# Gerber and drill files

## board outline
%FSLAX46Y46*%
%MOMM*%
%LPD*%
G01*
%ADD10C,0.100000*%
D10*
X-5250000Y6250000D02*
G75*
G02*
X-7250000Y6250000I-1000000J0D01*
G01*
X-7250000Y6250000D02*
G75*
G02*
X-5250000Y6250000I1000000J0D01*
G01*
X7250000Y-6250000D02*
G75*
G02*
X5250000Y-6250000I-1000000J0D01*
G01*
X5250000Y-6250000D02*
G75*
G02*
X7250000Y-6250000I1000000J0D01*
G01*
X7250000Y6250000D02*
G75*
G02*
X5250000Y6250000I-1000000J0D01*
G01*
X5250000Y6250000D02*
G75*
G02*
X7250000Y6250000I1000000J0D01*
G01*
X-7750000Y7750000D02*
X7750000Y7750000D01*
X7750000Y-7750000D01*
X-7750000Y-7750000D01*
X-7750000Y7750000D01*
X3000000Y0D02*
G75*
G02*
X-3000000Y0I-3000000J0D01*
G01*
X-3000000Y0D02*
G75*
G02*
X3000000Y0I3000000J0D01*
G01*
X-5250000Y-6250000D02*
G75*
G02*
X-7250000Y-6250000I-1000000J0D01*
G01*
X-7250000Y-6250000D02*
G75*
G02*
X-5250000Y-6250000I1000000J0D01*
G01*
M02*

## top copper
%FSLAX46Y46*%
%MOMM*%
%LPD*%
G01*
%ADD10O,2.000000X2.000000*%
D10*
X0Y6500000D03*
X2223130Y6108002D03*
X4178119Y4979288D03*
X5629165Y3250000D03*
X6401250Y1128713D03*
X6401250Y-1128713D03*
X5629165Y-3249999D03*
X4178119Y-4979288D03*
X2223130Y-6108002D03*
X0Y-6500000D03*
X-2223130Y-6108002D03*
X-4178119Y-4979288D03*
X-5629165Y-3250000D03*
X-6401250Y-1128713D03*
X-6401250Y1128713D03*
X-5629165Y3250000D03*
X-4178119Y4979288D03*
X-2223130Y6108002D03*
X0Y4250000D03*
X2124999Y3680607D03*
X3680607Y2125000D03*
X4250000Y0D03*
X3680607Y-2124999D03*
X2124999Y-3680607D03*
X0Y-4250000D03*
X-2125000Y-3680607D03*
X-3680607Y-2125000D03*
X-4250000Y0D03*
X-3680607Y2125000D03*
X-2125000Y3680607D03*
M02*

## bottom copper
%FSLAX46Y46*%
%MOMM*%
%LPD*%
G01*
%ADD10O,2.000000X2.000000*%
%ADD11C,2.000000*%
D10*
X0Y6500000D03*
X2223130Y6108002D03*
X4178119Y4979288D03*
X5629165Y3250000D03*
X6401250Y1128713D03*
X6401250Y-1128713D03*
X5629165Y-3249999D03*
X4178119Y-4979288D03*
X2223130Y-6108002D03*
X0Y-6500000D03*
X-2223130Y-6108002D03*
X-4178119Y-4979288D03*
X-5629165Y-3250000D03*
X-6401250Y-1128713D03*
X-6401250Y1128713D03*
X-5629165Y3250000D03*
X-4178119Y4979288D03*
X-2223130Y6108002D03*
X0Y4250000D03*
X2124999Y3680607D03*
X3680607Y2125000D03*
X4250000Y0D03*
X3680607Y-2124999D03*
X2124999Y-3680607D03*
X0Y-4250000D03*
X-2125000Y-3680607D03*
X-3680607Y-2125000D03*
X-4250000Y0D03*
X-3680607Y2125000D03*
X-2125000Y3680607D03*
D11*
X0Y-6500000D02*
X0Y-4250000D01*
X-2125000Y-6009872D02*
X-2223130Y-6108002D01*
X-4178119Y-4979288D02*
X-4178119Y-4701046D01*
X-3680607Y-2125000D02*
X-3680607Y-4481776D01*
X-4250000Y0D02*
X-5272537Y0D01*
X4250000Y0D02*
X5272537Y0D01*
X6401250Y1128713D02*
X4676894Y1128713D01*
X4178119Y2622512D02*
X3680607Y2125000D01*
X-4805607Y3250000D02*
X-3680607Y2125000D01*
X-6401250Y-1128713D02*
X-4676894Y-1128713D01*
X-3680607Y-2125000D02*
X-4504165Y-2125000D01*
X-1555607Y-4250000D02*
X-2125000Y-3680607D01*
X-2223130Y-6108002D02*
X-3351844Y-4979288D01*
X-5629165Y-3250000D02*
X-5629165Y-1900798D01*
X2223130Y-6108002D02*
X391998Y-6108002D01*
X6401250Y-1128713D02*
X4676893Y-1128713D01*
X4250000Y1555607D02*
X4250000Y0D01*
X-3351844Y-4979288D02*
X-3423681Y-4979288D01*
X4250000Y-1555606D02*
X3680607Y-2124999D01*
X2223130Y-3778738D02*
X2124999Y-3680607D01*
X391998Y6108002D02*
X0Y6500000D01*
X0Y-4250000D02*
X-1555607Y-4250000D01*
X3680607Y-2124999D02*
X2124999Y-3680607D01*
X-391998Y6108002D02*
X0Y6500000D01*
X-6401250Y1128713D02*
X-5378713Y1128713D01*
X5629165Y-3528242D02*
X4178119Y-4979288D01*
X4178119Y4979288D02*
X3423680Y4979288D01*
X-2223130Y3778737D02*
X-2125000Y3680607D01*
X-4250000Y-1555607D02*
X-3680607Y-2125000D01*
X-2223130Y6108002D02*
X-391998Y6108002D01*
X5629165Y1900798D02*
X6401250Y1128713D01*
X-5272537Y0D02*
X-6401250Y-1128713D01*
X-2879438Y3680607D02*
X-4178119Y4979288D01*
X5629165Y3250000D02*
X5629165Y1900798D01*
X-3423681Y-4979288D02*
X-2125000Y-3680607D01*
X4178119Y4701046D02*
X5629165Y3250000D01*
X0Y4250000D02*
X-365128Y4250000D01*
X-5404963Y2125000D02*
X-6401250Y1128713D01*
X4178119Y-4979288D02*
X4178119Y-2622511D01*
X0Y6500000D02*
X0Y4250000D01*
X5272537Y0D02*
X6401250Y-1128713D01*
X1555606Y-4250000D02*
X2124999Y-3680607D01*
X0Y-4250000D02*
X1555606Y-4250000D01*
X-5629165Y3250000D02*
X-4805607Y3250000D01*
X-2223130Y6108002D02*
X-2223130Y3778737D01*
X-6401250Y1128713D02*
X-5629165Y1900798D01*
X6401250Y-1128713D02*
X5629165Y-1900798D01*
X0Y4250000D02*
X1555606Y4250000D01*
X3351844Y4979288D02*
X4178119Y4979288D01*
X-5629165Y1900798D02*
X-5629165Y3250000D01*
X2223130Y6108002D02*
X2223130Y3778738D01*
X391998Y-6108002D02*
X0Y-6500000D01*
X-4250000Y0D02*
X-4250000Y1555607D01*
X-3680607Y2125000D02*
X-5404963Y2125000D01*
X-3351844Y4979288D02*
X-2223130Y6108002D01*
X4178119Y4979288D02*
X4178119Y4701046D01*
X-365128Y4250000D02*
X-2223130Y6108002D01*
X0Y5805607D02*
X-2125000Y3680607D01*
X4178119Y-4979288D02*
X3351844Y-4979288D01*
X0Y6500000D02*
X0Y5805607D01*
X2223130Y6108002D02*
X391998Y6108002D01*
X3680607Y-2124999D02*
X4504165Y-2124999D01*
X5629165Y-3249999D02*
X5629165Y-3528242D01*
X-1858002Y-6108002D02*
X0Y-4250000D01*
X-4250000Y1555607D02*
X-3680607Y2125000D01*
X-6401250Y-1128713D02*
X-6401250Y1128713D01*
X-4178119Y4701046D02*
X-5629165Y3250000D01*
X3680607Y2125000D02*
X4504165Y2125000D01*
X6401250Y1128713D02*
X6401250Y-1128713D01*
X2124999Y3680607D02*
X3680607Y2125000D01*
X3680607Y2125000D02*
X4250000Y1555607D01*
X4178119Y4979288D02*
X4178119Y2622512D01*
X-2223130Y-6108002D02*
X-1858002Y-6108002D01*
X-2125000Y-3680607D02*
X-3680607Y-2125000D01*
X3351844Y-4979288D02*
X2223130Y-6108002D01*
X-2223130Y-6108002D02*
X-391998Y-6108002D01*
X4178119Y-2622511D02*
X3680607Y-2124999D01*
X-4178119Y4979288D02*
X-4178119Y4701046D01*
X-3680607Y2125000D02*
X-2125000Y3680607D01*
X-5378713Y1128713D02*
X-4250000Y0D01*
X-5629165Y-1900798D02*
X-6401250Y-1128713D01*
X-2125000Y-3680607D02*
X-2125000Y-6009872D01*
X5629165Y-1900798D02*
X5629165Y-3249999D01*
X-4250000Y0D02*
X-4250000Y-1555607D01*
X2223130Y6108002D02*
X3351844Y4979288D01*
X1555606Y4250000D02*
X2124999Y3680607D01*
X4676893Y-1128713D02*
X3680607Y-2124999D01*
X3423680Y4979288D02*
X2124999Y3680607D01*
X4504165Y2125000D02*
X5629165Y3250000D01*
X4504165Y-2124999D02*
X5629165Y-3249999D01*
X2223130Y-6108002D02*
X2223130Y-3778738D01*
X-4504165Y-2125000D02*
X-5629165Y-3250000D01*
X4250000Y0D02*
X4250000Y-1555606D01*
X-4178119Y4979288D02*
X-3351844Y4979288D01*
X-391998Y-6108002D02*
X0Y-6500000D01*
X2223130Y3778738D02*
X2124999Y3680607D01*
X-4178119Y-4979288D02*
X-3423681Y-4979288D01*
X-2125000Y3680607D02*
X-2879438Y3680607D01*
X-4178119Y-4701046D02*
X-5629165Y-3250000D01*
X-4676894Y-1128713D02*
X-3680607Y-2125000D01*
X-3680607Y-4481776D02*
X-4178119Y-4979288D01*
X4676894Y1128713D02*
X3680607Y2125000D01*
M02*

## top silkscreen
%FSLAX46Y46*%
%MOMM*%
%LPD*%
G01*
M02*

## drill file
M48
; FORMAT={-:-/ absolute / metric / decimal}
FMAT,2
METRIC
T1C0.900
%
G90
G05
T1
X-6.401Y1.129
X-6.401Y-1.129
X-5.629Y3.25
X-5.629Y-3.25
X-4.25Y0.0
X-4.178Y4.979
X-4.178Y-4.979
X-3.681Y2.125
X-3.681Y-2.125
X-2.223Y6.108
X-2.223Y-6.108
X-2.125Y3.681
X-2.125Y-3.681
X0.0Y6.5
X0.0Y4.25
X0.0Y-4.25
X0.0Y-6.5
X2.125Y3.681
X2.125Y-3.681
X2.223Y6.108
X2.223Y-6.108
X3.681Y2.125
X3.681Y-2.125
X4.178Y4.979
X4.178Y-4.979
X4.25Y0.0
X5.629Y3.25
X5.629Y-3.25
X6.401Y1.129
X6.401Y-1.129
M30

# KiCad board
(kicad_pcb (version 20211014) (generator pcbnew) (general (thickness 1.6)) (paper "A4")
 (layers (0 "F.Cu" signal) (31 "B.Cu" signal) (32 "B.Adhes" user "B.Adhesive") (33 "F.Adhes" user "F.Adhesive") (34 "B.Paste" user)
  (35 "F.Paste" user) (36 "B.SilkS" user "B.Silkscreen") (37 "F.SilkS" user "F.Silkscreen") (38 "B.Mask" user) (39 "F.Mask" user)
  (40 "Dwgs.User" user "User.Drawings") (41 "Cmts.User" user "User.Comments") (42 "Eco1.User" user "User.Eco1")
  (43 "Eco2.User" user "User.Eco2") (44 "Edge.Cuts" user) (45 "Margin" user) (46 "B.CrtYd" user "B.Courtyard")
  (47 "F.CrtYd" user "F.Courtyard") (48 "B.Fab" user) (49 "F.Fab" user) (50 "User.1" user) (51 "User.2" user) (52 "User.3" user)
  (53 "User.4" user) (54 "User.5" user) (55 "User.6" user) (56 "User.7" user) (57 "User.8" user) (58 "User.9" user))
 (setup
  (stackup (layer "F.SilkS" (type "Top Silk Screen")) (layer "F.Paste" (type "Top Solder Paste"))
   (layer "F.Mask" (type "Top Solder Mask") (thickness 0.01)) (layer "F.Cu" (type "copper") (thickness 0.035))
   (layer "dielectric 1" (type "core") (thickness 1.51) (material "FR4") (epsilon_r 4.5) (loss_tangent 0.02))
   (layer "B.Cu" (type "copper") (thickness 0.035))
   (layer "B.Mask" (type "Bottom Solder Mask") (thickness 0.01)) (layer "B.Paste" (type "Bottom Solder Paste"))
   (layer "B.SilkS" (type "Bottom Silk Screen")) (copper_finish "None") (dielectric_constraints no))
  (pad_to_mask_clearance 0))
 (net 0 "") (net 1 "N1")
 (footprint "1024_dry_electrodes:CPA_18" (layer "F.Cu") (at 0 0)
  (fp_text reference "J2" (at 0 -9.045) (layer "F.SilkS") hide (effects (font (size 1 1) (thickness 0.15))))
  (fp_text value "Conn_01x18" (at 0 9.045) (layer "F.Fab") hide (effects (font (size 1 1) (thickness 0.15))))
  (pad "1" thru_hole oval (at 0 -6.5) (size 2 2) (drill 0.9) (layers *.Cu *.Mask) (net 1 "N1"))
  (pad "2" thru_hole oval (at 2.22313 -6.108002) (size 2 2) (drill 0.9) (layers *.Cu *.Mask) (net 1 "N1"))
  (pad "3" thru_hole oval (at 4.178119 -4.979288) (size 2 2) (drill 0.9) (layers *.Cu *.Mask) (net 1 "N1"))
  (pad "4" thru_hole oval (at 5.629165 -3.25) (size 2 2) (drill 0.9) (layers *.Cu *.Mask) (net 1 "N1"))
  (pad "5" thru_hole oval (at 6.40125 -1.128713) (size 2 2) (drill 0.9) (layers *.Cu *.Mask) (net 1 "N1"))
  (pad "6" thru_hole oval (at 6.40125 1.128713) (size 2 2) (drill 0.9) (layers *.Cu *.Mask) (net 1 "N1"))
  (pad "7" thru_hole oval (at 5.629165 3.249999) (size 2 2) (drill 0.9) (layers *.Cu *.Mask) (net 1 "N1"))
  (pad "8" thru_hole oval (at 4.178119 4.979288) (size 2 2) (drill 0.9) (layers *.Cu *.Mask) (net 1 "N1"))
  (pad "9" thru_hole oval (at 2.22313 6.108002) (size 2 2) (drill 0.9) (layers *.Cu *.Mask) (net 1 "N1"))
  (pad "10" thru_hole oval (at 0 6.5) (size 2 2) (drill 0.9) (layers *.Cu *.Mask) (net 1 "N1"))
  (pad "11" thru_hole oval (at -2.22313 6.108002) (size 2 2) (drill 0.9) (layers *.Cu *.Mask) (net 1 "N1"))
  (pad "12" thru_hole oval (at -4.178119 4.979288) (size 2 2) (drill 0.9) (layers *.Cu *.Mask) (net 1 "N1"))
  (pad "13" thru_hole oval (at -5.629165 3.25) (size 2 2) (drill 0.9) (layers *.Cu *.Mask) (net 1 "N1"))
  (pad "14" thru_hole oval (at -6.40125 1.128713) (size 2 2) (drill 0.9) (layers *.Cu *.Mask) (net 1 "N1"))
  (pad "15" thru_hole oval (at -6.40125 -1.128713) (size 2 2) (drill 0.9) (layers *.Cu *.Mask) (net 1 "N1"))
  (pad "16" thru_hole oval (at -5.629165 -3.25) (size 2 2) (drill 0.9) (layers *.Cu *.Mask) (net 1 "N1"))
  (pad "17" thru_hole oval (at -4.178119 -4.979288) (size 2 2) (drill 0.9) (layers *.Cu *.Mask) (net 1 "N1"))
  (pad "18" thru_hole oval (at -2.22313 -6.108002) (size 2 2) (drill 0.9) (layers *.Cu *.Mask) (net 1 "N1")))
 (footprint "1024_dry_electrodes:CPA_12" (layer "F.Cu") (at 0 0)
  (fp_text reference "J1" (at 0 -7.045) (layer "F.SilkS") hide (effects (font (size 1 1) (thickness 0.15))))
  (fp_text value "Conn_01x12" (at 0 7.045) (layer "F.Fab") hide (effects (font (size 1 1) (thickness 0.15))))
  (pad "1" thru_hole oval (at 0 -4.25) (size 2 2) (drill 0.9) (layers *.Cu *.Mask) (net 1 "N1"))
  (pad "2" thru_hole oval (at 2.124999 -3.680607) (size 2 2) (drill 0.9) (layers *.Cu *.Mask) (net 1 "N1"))
  (pad "3" thru_hole oval (at 3.680607 -2.125) (size 2 2) (drill 0.9) (layers *.Cu *.Mask) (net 1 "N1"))
  (pad "4" thru_hole oval (at 4.25 0) (size 2 2) (drill 0.9) (layers *.Cu *.Mask) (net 1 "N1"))
  (pad "5" thru_hole oval (at 3.680607 2.124999) (size 2 2) (drill 0.9) (layers *.Cu *.Mask) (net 1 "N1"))
  (pad "6" thru_hole oval (at 2.124999 3.680607) (size 2 2) (drill 0.9) (layers *.Cu *.Mask) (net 1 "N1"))
  (pad "7" thru_hole oval (at 0 4.25) (size 2 2) (drill 0.9) (layers *.Cu *.Mask) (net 1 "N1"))
  (pad "8" thru_hole oval (at -2.125 3.680607) (size 2 2) (drill 0.9) (layers *.Cu *.Mask) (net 1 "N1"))
  (pad "9" thru_hole oval (at -3.680607 2.125) (size 2 2) (drill 0.9) (layers *.Cu *.Mask) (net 1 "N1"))
  (pad "10" thru_hole oval (at -4.25 0) (size 2 2) (drill 0.9) (layers *.Cu *.Mask) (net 1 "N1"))
  (pad "11" thru_hole oval (at -3.680607 -2.125) (size 2 2) (drill 0.9) (layers *.Cu *.Mask) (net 1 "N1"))
  (pad "12" thru_hole oval (at -2.125 -3.680607) (size 2 2) (drill 0.9) (layers *.Cu *.Mask) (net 1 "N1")))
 (gr_circle (center -6.25 -6.25) (end -5.25 -6.25) (layer "Edge.Cuts") (width 0.1) (fill none))
 (gr_circle (center 6.25 6.25) (end 7.25 6.25) (layer "Edge.Cuts") (width 0.1) (fill none))
 (gr_circle (center 6.25 -6.25) (end 7.25 -6.25) (layer "Edge.Cuts") (width 0.1) (fill none))
 (gr_rect (start 7.75 7.75) (end -7.75 -7.75) (layer "Edge.Cuts") (width 0.1) (fill none))
 (gr_circle (center 0 0) (end 3 0) (layer "Edge.Cuts") (width 0.1) (fill none))
 (gr_circle (center -6.25 6.25) (end -5.25 6.25) (layer "Edge.Cuts") (width 0.1) (fill none))
 (segment (start 0 6.5) (end 0 4.25) (width 2) (layer "B.Cu") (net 1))
 (segment (start -2.125 6.009872) (end -2.22313 6.108002) (width 2) (layer "B.Cu") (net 1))
 (segment (start -4.178119 4.979288) (end -4.178119 4.701046) (width 2) (layer "B.Cu") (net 1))
 (segment (start -3.680607 2.125) (end -3.680607 4.481776) (width 2) (layer "B.Cu") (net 1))
 (segment (start -4.25 0) (end -5.272537 0) (width 2) (layer "B.Cu") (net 1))
 (segment (start 4.25 0) (end 5.272537 0) (width 2) (layer "B.Cu") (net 1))
 (segment (start 6.40125 -1.128713) (end 4.676894 -1.128713) (width 2) (layer "B.Cu") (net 1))
 (segment (start 4.178119 -2.622512) (end 3.680607 -2.125) (width 2) (layer "B.Cu") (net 1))
 (segment (start -4.805607 -3.25) (end -3.680607 -2.125) (width 2) (layer "B.Cu") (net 1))
 (segment (start -6.40125 1.128713) (end -4.676894 1.128713) (width 2) (layer "B.Cu") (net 1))
 (segment (start -3.680607 2.125) (end -4.504165 2.125) (width 2) (layer "B.Cu") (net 1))
 (segment (start -1.555607 4.25) (end -2.125 3.680607) (width 2) (layer "B.Cu") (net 1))
 (segment (start -2.22313 6.108002) (end -3.351844 4.979288) (width 2) (layer "B.Cu") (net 1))
 (segment (start -5.629165 3.25) (end -5.629165 1.900798) (width 2) (layer "B.Cu") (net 1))
 (segment (start 2.22313 6.108002) (end 0.391998 6.108002) (width 2) (layer "B.Cu") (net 1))
 (segment (start 6.40125 1.128713) (end 4.676893 1.128713) (width 2) (layer "B.Cu") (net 1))
 (segment (start 4.25 -1.555607) (end 4.25 0) (width 2) (layer "B.Cu") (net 1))
 (segment (start -3.351844 4.979288) (end -3.423681 4.979288) (width 2) (layer "B.Cu") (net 1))
 (segment (start 4.25 1.555606) (end 3.680607 2.124999) (width 2) (layer "B.Cu") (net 1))
 (segment (start 2.22313 3.778738) (end 2.124999 3.680607) (width 2) (layer "B.Cu") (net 1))
 (segment (start 0.391998 -6.108002) (end 0 -6.5) (width 2) (layer "B.Cu") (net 1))
 (segment (start 0 4.25) (end -1.555607 4.25) (width 2) (layer "B.Cu") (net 1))
 (segment (start 3.680607 2.124999) (end 2.124999 3.680607) (width 2) (layer "B.Cu") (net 1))
 (segment (start -0.391998 -6.108002) (end 0 -6.5) (width 2) (layer "B.Cu") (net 1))
 (segment (start -6.40125 -1.128713) (end -5.378713 -1.128713) (width 2) (layer "B.Cu") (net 1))
 (segment (start 5.629165 3.528242) (end 4.178119 4.979288) (width 2) (layer "B.Cu") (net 1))
 (segment (start 4.178119 -4.979288) (end 3.42368 -4.979288) (width 2) (layer "B.Cu") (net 1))
 (segment (start -2.22313 -3.778737) (end -2.125 -3.680607) (width 2) (layer "B.Cu") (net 1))
 (segment (start -4.25 1.555607) (end -3.680607 2.125) (width 2) (layer "B.Cu") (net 1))
 (segment (start -2.22313 -6.108002) (end -0.391998 -6.108002) (width 2) (layer "B.Cu") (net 1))
 (segment (start 5.629165 -1.900798) (end 6.40125 -1.128713) (width 2) (layer "B.Cu") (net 1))
 (segment (start -5.272537 0) (end -6.40125 1.128713) (width 2) (layer "B.Cu") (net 1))
 (segment (start -2.879438 -3.680607) (end -4.178119 -4.979288) (width 2) (layer "B.Cu") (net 1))
 (segment (start 5.629165 -3.25) (end 5.629165 -1.900798) (width 2) (layer "B.Cu") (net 1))
 (segment (start -3.423681 4.979288) (end -2.125 3.680607) (width 2) (layer "B.Cu") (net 1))
 (segment (start 4.178119 -4.701046) (end 5.629165 -3.25) (width 2) (layer "B.Cu") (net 1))
 (segment (start 0 -4.25) (end -0.365128 -4.25) (width 2) (layer "B.Cu") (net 1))
 (segment (start -5.404963 -2.125) (end -6.40125 -1.128713) (width 2) (layer "B.Cu") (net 1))
 (segment (start 4.178119 4.979288) (end 4.178119 2.622511) (width 2) (layer "B.Cu") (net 1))
 (segment (start 0 -6.5) (end 0 -4.25) (width 2) (layer "B.Cu") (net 1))
 (segment (start 5.272537 0) (end 6.40125 1.128713) (width 2) (layer "B.Cu") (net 1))
 (segment (start 1.555606 4.25) (end 2.124999 3.680607) (width 2) (layer "B.Cu") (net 1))
 (segment (start 0 4.25) (end 1.555606 4.25) (width 2) (layer "B.Cu") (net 1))
 (segment (start -5.629165 -3.25) (end -4.805607 -3.25) (width 2) (layer "B.Cu") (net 1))
 (segment (start -2.22313 -6.108002) (end -2.22313 -3.778737) (width 2) (layer "B.Cu") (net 1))
 (segment (start -6.40125 -1.128713) (end -5.629165 -1.900798) (width 2) (layer "B.Cu") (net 1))
 (segment (start 6.40125 1.128713) (end 5.629165 1.900798) (width 2) (layer "B.Cu") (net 1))
 (segment (start 0 -4.25) (end 1.555606 -4.25) (width 2) (layer "B.Cu") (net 1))
 (segment (start 3.351844 -4.979288) (end 4.178119 -4.979288) (width 2) (layer "B.Cu") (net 1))
 (segment (start -5.629165 -1.900798) (end -5.629165 -3.25) (width 2) (layer "B.Cu") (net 1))
 (segment (start 2.22313 -6.108002) (end 2.22313 -3.778738) (width 2) (layer "B.Cu") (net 1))
 (segment (start 0.391998 6.108002) (end 0 6.5) (width 2) (layer "B.Cu") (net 1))
 (segment (start -4.25 0) (end -4.25 -1.555607) (width 2) (layer "B.Cu") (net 1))
 (segment (start -3.680607 -2.125) (end -5.404963 -2.125) (width 2) (layer "B.Cu") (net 1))
 (segment (start -3.351844 -4.979288) (end -2.22313 -6.108002) (width 2) (layer "B.Cu") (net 1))
 (segment (start 4.178119 -4.979288) (end 4.178119 -4.701046) (width 2) (layer "B.Cu") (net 1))
 (segment (start -0.365128 -4.25) (end -2.22313 -6.108002) (width 2) (layer "B.Cu") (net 1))
 (segment (start 0 -5.805607) (end -2.125 -3.680607) (width 2) (layer "B.Cu") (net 1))
 (segment (start 4.178119 4.979288) (end 3.351844 4.979288) (width 2) (layer "B.Cu") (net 1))
 (segment (start 0 -6.5) (end 0 -5.805607) (width 2) (layer "B.Cu") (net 1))
 (segment (start 2.22313 -6.108002) (end 0.391998 -6.108002) (width 2) (layer "B.Cu") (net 1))
 (segment (start 3.680607 2.124999) (end 4.504165 2.124999) (width 2) (layer "B.Cu") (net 1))
 (segment (start 5.629165 3.249999) (end 5.629165 3.528242) (width 2) (layer "B.Cu") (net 1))
 (segment (start -1.858002 6.108002) (end 0 4.25) (width 2) (layer "B.Cu") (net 1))
 (segment (start -4.25 -1.555607) (end -3.680607 -2.125) (width 2) (layer "B.Cu") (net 1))
 (segment (start -6.40125 1.128713) (end -6.40125 -1.128713) (width 2) (layer "B.Cu") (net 1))
 (segment (start -4.178119 -4.701046) (end -5.629165 -3.25) (width 2) (layer "B.Cu") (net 1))
 (segment (start 3.680607 -2.125) (end 4.504165 -2.125) (width 2) (layer "B.Cu") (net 1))
 (segment (start 6.40125 -1.128713) (end 6.40125 1.128713) (width 2) (layer "B.Cu") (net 1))
 (segment (start 2.124999 -3.680607) (end 3.680607 -2.125) (width 2) (layer "B.Cu") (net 1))
 (segment (start 3.680607 -2.125) (end 4.25 -1.555607) (width 2) (layer "B.Cu") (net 1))
 (segment (start 4.178119 -4.979288) (end 4.178119 -2.622512) (width 2) (layer "B.Cu") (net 1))
 (segment (start -2.22313 6.108002) (end -1.858002 6.108002) (width 2) (layer "B.Cu") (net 1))
 (segment (start -2.125 3.680607) (end -3.680607 2.125) (width 2) (layer "B.Cu") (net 1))
 (segment (start 3.351844 4.979288) (end 2.22313 6.108002) (width 2) (layer "B.Cu") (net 1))
 (segment (start -2.22313 6.108002) (end -0.391998 6.108002) (width 2) (layer "B.Cu") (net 1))
 (segment (start 4.178119 2.622511) (end 3.680607 2.124999) (width 2) (layer "B.Cu") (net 1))
 (segment (start -4.178119 -4.979288) (end -4.178119 -4.701046) (width 2) (layer "B.Cu") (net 1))
 (segment (start -3.680607 -2.125) (end -2.125 -3.680607) (width 2) (layer "B.Cu") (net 1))
 (segment (start -5.378713 -1.128713) (end -4.25 0) (width 2) (layer "B.Cu") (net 1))
 (segment (start -5.629165 1.900798) (end -6.40125 1.128713) (width 2) (layer "B.Cu") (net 1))
 (segment (start -2.125 3.680607) (end -2.125 6.009872) (width 2) (layer "B.Cu") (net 1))
 (segment (start 5.629165 1.900798) (end 5.629165 3.249999) (width 2) (layer "B.Cu") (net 1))
 (segment (start -4.25 0) (end -4.25 1.555607) (width 2) (layer "B.Cu") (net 1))
 (segment (start 2.22313 -6.108002) (end 3.351844 -4.979288) (width 2) (layer "B.Cu") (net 1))
 (segment (start 1.555606 -4.25) (end 2.124999 -3.680607) (width 2) (layer "B.Cu") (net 1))
 (segment (start 4.676893 1.128713) (end 3.680607 2.124999) (width 2) (layer "B.Cu") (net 1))
 (segment (start 3.42368 -4.979288) (end 2.124999 -3.680607) (width 2) (layer "B.Cu") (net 1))
 (segment (start 4.504165 -2.125) (end 5.629165 -3.25) (width 2) (layer "B.Cu") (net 1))
 (segment (start 4.504165 2.124999) (end 5.629165 3.249999) (width 2) (layer "B.Cu") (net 1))
 (segment (start 2.22313 6.108002) (end 2.22313 3.778738) (width 2) (layer "B.Cu") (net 1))
 (segment (start -4.504165 2.125) (end -5.629165 3.25) (width 2) (layer "B.Cu") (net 1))
 (segment (start 4.25 0) (end 4.25 1.555606) (width 2) (layer "B.Cu") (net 1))
 (segment (start -4.178119 -4.979288) (end -3.351844 -4.979288) (width 2) (layer "B.Cu") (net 1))
 (segment (start -0.391998 6.108002) (end 0 6.5) (width 2) (layer "B.Cu") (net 1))
 (segment (start 2.22313 -3.778738) (end 2.124999 -3.680607) (width 2) (layer "B.Cu") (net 1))
 (segment (start -4.178119 4.979288) (end -3.423681 4.979288) (width 2) (layer "B.Cu") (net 1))
 (segment (start -2.125 -3.680607) (end -2.879438 -3.680607) (width 2) (layer "B.Cu") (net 1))
 (segment (start -4.178119 4.701046) (end -5.629165 3.25) (width 2) (layer "B.Cu") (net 1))
 (segment (start -4.676894 1.128713) (end -3.680607 2.125) (width 2) (layer "B.Cu") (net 1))
 (segment (start -3.680607 4.481776) (end -4.178119 4.979288) (width 2) (layer "B.Cu") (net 1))
 (segment (start 4.676894 -1.128713) (end 3.680607 -2.125) (width 2) (layer "B.Cu") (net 1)))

